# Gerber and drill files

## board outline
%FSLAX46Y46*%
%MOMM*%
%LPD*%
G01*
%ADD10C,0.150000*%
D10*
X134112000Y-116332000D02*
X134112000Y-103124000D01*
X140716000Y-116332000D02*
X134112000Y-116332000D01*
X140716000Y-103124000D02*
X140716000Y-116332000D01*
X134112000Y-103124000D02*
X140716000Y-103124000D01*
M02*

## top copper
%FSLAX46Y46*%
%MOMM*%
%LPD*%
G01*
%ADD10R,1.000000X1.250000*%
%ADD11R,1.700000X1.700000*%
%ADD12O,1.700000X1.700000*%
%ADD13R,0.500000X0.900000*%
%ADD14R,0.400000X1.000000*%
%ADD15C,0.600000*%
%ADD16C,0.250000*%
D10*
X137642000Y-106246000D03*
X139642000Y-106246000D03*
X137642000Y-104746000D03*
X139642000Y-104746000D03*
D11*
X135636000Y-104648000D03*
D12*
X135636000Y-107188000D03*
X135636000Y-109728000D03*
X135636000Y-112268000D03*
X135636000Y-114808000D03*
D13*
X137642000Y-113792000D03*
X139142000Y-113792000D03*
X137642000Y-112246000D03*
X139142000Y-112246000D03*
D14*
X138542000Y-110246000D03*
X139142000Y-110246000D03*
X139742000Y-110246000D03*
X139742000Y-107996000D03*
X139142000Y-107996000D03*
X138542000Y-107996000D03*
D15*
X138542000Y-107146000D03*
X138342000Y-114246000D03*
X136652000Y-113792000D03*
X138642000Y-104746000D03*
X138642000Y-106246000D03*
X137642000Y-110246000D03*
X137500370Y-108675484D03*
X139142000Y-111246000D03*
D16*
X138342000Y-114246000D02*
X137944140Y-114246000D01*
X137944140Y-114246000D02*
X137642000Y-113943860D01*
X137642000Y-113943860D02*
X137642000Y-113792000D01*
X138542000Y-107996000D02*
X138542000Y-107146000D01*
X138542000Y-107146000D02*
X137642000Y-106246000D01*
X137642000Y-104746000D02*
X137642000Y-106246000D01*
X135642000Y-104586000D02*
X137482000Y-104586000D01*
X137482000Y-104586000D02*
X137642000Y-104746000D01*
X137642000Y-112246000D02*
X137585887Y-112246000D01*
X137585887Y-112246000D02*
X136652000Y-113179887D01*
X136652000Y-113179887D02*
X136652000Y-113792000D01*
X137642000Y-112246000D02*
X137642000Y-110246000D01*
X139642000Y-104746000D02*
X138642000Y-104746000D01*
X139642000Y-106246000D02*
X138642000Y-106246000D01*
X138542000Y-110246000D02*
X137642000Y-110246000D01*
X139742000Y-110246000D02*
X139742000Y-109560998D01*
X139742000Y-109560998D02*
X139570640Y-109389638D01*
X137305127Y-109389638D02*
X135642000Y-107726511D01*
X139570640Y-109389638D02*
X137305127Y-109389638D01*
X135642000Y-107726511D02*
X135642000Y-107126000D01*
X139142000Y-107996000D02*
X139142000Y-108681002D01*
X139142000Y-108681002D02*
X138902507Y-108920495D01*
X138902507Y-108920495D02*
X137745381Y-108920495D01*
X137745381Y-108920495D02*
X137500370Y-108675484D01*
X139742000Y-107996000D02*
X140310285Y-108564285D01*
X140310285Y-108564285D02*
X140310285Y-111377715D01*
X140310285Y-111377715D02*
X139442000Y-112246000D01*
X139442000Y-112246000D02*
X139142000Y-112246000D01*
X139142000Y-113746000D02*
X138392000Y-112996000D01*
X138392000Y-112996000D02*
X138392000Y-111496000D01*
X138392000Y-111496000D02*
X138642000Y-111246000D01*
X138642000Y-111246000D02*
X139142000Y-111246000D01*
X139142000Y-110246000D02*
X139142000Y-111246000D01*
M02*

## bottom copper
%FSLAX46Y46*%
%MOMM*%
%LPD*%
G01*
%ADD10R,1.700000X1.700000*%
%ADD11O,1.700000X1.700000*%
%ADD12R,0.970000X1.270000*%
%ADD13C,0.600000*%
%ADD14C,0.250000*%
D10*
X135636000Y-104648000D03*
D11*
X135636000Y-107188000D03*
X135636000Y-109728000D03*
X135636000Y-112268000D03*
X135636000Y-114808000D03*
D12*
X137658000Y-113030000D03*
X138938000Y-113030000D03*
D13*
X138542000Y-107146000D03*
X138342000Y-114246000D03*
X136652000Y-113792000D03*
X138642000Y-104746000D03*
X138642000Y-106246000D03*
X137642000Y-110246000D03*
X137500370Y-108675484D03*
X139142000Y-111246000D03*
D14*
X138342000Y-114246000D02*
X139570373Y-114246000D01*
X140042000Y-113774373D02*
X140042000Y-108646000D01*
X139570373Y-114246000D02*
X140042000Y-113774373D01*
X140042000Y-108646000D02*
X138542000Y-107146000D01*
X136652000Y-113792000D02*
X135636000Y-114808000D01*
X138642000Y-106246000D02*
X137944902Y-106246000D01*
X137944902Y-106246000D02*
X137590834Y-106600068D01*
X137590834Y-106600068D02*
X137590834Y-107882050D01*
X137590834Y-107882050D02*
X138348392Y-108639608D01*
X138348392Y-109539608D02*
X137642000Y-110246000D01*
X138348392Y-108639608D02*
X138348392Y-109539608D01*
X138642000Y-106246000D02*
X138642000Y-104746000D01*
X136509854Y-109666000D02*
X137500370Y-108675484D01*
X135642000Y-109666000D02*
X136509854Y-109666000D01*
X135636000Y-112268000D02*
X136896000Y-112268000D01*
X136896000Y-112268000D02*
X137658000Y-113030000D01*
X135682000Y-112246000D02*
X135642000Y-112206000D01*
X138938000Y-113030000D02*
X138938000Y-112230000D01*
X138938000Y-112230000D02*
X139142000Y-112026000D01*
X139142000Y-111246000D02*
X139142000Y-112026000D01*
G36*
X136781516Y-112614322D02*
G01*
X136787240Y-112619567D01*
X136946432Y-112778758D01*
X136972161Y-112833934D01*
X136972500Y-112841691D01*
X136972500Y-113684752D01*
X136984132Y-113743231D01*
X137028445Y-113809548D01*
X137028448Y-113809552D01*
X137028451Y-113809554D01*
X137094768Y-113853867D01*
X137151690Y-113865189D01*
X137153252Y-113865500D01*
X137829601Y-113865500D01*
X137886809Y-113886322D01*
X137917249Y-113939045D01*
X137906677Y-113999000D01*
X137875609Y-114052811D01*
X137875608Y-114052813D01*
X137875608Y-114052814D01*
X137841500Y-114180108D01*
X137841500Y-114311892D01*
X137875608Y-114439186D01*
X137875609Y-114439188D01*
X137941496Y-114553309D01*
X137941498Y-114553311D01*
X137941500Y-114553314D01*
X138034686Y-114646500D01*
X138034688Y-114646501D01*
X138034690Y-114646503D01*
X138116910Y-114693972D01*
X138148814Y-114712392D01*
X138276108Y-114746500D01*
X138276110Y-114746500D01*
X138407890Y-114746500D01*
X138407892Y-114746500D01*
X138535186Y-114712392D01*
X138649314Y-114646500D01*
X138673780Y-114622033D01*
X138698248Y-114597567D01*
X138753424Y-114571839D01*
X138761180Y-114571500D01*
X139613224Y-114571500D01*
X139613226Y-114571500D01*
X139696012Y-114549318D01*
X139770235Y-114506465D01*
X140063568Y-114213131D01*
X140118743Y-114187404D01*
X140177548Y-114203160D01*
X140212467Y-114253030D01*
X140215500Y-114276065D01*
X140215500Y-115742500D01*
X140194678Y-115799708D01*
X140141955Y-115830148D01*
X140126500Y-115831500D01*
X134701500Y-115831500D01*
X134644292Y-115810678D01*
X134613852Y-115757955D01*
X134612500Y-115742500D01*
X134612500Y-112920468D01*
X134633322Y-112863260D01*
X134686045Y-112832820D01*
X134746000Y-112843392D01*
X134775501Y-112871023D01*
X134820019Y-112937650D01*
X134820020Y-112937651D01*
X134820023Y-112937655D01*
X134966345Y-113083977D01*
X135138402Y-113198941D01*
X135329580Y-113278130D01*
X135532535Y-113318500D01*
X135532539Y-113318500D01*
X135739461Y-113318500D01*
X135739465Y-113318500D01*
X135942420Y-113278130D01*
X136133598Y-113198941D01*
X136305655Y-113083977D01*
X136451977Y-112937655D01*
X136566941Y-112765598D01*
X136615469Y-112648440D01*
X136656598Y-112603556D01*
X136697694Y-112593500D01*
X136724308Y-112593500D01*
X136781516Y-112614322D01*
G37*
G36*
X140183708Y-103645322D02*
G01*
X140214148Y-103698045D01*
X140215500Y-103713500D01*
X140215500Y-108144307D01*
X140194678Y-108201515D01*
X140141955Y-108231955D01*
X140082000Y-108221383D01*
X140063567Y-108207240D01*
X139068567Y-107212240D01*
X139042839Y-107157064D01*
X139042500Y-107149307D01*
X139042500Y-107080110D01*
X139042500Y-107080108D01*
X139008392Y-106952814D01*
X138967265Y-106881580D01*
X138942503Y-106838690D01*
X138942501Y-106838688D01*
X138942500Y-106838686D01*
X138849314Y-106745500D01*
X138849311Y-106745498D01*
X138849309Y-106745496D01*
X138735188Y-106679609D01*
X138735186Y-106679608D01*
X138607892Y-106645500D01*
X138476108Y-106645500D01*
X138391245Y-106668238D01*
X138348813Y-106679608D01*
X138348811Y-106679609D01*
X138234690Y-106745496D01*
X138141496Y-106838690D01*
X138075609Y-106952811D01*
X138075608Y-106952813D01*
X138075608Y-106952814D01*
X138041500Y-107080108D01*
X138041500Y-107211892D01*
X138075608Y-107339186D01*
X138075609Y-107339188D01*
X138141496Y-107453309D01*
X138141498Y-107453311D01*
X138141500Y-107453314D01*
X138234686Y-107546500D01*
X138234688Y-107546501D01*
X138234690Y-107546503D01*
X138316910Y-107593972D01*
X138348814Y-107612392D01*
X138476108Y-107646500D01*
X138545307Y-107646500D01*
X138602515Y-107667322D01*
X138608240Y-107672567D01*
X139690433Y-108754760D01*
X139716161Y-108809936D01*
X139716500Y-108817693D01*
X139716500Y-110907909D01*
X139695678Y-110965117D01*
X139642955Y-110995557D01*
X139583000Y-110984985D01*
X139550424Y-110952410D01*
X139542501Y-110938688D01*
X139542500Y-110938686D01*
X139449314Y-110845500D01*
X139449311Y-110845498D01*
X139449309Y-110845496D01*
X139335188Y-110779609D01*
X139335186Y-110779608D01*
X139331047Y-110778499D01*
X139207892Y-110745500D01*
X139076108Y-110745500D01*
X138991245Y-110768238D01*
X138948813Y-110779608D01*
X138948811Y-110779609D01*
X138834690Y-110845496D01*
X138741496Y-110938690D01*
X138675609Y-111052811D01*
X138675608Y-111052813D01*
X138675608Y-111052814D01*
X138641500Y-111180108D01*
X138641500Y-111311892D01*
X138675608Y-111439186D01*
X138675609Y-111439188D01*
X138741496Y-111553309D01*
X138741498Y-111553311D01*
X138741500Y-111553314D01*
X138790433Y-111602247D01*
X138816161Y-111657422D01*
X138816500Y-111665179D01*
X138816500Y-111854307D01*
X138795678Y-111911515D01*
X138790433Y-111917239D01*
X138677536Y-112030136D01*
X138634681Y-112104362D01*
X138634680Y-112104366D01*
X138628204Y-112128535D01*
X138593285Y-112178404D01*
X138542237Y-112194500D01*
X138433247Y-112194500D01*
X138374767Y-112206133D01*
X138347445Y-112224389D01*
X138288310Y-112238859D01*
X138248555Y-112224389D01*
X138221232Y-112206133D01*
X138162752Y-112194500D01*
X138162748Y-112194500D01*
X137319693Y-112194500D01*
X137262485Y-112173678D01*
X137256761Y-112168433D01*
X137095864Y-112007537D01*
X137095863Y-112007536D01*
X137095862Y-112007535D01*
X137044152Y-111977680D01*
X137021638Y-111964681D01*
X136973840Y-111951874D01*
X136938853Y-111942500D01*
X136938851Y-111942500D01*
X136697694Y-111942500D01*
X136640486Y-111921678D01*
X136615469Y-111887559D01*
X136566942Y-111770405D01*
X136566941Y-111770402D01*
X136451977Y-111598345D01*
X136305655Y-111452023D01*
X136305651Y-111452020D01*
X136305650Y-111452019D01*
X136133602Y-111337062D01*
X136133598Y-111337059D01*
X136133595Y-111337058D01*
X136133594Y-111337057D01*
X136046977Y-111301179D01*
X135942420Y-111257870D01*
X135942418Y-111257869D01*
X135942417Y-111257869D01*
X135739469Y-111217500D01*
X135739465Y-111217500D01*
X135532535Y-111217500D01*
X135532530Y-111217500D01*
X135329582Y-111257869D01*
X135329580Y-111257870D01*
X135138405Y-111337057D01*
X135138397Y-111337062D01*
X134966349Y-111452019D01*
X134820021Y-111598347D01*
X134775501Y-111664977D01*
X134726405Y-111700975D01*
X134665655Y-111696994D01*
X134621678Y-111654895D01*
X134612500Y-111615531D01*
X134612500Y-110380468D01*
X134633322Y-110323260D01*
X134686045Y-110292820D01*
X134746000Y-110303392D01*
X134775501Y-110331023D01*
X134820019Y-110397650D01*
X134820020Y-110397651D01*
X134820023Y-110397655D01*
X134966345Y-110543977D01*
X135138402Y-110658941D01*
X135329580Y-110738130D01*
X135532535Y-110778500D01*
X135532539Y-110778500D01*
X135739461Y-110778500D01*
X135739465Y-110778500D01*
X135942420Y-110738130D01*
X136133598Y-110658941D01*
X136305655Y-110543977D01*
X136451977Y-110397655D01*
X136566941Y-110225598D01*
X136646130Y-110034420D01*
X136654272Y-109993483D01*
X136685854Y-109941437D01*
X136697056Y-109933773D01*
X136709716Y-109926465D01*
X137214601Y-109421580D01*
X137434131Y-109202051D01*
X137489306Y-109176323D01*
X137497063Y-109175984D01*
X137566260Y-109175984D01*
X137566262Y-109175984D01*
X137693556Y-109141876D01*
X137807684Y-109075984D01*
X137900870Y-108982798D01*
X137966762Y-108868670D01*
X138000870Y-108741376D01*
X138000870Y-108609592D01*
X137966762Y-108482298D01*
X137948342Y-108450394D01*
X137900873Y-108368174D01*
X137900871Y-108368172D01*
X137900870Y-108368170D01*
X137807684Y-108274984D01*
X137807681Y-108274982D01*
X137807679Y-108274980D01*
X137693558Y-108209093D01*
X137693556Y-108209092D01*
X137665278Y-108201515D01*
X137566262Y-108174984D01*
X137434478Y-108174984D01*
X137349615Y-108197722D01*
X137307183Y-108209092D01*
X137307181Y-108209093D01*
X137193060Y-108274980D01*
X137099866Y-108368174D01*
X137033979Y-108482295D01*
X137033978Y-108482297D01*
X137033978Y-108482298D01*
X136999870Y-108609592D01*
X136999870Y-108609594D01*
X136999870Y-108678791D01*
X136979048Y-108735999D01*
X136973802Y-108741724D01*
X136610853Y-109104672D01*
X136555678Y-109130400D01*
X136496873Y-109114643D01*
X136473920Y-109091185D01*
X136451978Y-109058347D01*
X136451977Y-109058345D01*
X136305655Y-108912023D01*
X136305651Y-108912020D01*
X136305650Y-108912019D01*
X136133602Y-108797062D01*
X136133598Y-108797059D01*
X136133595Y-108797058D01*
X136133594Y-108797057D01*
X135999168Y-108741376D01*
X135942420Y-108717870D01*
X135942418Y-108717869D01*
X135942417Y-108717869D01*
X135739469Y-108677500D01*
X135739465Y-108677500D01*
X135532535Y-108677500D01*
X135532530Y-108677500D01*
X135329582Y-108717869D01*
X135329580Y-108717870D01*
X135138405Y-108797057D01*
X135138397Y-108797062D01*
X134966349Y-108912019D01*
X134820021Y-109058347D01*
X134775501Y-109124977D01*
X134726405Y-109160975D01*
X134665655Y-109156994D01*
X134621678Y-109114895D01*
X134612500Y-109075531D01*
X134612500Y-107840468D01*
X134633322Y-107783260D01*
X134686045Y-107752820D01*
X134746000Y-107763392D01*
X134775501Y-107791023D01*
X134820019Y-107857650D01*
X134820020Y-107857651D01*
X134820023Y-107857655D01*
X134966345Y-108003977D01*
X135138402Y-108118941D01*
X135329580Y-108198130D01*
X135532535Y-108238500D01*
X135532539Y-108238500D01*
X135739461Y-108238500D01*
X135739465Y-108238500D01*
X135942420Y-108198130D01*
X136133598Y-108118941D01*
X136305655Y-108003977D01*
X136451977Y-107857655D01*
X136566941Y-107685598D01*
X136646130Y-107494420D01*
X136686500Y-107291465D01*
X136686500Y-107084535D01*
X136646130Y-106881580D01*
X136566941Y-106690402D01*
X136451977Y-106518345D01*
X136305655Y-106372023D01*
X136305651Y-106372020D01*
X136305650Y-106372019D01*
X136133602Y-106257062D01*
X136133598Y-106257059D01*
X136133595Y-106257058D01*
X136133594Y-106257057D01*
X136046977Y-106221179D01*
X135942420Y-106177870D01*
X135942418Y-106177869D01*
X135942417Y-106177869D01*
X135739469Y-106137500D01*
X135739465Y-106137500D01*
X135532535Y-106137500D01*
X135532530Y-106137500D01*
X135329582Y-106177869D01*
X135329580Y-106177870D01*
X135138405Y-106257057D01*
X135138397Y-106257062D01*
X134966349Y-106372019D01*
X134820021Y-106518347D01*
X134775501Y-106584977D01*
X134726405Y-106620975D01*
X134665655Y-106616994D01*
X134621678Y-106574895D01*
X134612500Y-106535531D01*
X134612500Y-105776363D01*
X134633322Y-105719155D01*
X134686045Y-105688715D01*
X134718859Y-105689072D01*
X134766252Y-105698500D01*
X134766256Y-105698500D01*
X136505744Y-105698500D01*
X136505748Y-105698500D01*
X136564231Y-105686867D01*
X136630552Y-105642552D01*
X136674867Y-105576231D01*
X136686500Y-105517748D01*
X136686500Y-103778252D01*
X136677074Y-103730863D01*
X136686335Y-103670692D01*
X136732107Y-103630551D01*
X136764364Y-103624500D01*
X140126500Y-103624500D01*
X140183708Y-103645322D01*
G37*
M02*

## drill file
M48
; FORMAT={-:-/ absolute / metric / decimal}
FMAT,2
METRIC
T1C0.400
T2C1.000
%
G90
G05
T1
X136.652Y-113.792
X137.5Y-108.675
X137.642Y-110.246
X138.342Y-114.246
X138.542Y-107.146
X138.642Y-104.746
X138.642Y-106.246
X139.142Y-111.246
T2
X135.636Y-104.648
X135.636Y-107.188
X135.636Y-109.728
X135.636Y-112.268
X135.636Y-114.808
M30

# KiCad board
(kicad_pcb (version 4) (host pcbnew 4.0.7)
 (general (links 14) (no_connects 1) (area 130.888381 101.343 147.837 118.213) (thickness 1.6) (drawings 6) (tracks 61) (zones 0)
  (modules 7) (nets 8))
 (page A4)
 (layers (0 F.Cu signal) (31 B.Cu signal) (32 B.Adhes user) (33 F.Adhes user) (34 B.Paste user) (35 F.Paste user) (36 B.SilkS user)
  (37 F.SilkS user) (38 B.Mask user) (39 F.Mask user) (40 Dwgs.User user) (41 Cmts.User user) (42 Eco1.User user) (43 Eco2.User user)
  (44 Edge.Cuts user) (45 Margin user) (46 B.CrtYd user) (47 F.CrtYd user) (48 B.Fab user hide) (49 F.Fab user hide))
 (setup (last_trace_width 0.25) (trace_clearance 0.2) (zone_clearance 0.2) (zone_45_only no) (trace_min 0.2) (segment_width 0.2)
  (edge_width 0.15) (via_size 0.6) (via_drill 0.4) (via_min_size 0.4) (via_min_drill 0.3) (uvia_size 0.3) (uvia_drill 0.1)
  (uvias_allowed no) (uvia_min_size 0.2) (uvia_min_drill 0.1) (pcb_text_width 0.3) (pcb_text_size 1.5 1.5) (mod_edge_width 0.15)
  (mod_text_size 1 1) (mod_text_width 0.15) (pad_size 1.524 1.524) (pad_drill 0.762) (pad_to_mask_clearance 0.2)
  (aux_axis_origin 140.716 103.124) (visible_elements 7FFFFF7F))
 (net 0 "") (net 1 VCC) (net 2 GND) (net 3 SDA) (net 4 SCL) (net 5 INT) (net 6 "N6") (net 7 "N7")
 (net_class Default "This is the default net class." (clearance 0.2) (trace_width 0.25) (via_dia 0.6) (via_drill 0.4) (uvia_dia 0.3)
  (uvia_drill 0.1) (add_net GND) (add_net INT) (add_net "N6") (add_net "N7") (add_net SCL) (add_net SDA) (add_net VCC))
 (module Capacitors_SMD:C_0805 (layer F.Cu) (at 138.642 106.246)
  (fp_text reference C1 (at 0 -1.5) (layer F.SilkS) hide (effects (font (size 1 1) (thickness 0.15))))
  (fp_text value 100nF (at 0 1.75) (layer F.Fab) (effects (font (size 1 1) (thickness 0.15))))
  (pad 1 smd rect (at -1 0) (size 1 1.25) (layers F.Cu F.Paste F.Mask) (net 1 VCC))
  (pad 2 smd rect (at 1 0) (size 1 1.25) (layers F.Cu F.Paste F.Mask) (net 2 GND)))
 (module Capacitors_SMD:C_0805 (layer F.Cu) (at 138.642 104.746)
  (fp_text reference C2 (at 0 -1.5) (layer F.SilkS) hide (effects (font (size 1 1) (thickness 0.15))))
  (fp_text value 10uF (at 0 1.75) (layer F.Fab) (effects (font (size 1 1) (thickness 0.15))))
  (pad 1 smd rect (at -1 0) (size 1 1.25) (layers F.Cu F.Paste F.Mask) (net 1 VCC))
  (pad 2 smd rect (at 1 0) (size 1 1.25) (layers F.Cu F.Paste F.Mask) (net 2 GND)))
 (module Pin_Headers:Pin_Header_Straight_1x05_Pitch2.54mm (layer F.Cu) (at 135.636 104.648)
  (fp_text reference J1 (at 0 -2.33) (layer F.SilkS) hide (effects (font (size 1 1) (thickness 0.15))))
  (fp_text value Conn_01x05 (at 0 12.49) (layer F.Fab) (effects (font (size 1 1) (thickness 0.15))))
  (pad 1 thru_hole rect (at 0 0) (size 1.7 1.7) (drill 1) (layers *.Cu *.Mask) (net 1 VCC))
  (pad 2 thru_hole oval (at 0 2.54) (size 1.7 1.7) (drill 1) (layers *.Cu *.Mask) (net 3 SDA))
  (pad 3 thru_hole oval (at 0 5.08) (size 1.7 1.7) (drill 1) (layers *.Cu *.Mask) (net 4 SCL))
  (pad 4 thru_hole oval (at 0 7.62) (size 1.7 1.7) (drill 1) (layers *.Cu *.Mask) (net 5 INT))
  (pad 5 thru_hole oval (at 0 10.16) (size 1.7 1.7) (drill 1) (layers *.Cu *.Mask) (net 2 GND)))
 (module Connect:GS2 (layer B.Cu) (at 138.298 113.03 270)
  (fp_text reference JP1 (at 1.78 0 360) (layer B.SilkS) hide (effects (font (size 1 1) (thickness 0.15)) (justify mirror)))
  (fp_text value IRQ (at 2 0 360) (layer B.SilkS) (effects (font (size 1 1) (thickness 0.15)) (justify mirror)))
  (pad 1 smd rect (at 0 0.64 270) (size 1.27 0.97) (layers B.Cu B.Paste B.Mask) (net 5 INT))
  (pad 2 smd rect (at 0 -0.64 270) (size 1.27 0.97) (layers B.Cu B.Paste B.Mask) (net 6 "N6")))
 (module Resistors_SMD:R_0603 (layer F.Cu) (at 138.392 113.792)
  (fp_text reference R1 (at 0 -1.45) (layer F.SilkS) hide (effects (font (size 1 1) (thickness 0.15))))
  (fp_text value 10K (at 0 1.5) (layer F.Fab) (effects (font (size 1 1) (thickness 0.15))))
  (pad 1 smd rect (at -0.75 0) (size 0.5 0.9) (layers F.Cu F.Paste F.Mask) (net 1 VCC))
  (pad 2 smd rect (at 0.75 0) (size 0.5 0.9) (layers F.Cu F.Paste F.Mask) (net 6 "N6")))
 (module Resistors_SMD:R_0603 (layer F.Cu) (at 138.392 112.246)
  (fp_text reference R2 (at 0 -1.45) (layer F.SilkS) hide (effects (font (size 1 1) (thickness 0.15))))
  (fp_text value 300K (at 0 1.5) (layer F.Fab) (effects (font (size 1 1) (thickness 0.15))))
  (pad 1 smd rect (at -0.75 0) (size 0.5 0.9) (layers F.Cu F.Paste F.Mask) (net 2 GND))
  (pad 2 smd rect (at 0.75 0) (size 0.5 0.9) (layers F.Cu F.Paste F.Mask) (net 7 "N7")))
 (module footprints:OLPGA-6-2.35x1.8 (layer F.Cu) (at 139.142 109.171 90)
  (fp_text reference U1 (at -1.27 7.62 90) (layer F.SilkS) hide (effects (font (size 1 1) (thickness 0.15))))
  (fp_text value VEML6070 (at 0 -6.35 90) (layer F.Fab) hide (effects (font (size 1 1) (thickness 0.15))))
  (pad 1 smd rect (at -1.075 -0.6 90) (size 1 0.4) (layers F.Cu F.Paste F.Mask) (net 2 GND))
  (pad 2 smd rect (at -1.075 0 90) (size 1 0.4) (layers F.Cu F.Paste F.Mask) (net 6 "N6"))
  (pad 3 smd rect (at -1.075 0.6 90) (size 1 0.4) (layers F.Cu F.Paste F.Mask) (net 3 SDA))
  (pad 4 smd rect (at 1.175 0.6 90) (size 1 0.4) (layers F.Cu F.Paste F.Mask) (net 7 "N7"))
  (pad 5 smd rect (at 1.175 0 90) (size 1 0.4) (layers F.Cu F.Paste F.Mask) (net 4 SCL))
  (pad 6 smd rect (at 1.175 -0.6 90) (size 1 0.4) (layers F.Cu F.Paste F.Mask) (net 1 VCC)))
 (gr_line (start 134.112 116.332) (end 134.112 103.124) (layer Edge.Cuts) (width 0.15))
 (gr_line (start 140.716 116.332) (end 134.112 116.332) (layer Edge.Cuts) (width 0.15))
 (gr_line (start 140.716 103.124) (end 140.716 116.332) (layer Edge.Cuts) (width 0.15))
 (gr_line (start 134.112 103.124) (end 140.716 103.124) (layer Edge.Cuts) (width 0.15))
 (segment (start 138.342 114.246) (end 137.94414 114.246) (width 0.25) (layer F.Cu) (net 1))
 (segment (start 137.94414 114.246) (end 137.642 113.94386) (width 0.25) (layer F.Cu) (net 1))
 (segment (start 137.642 113.94386) (end 137.642 113.792) (width 0.25) (layer F.Cu) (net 1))
 (segment (start 138.342 114.246) (end 139.570373 114.246) (width 0.25) (layer B.Cu) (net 1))
 (segment (start 140.042 113.774373) (end 140.042 108.646) (width 0.25) (layer B.Cu) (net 1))
 (segment (start 139.570373 114.246) (end 140.042 113.774373) (width 0.25) (layer B.Cu) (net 1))
 (segment (start 140.042 108.646) (end 138.542 107.146) (width 0.25) (layer B.Cu) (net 1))
 (via (at 138.542 107.146) (size 0.6) (drill 0.4) (layers F.Cu B.Cu) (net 1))
 (via (at 138.342 114.246) (size 0.6) (drill 0.4) (layers F.Cu B.Cu) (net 1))
 (segment (start 138.542 107.996) (end 138.542 107.146) (width 0.25) (layer F.Cu) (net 1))
 (segment (start 138.542 107.146) (end 137.642 106.246) (width 0.25) (layer F.Cu) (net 1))
 (segment (start 137.642 104.746) (end 137.642 106.246) (width 0.25) (layer F.Cu) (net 1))
 (segment (start 135.642 104.586) (end 137.482 104.586) (width 0.25) (layer F.Cu) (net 1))
 (segment (start 137.482 104.586) (end 137.642 104.746) (width 0.25) (layer F.Cu) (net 1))
 (segment (start 137.642 112.246) (end 137.585887 112.246) (width 0.25) (layer F.Cu) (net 2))
 (segment (start 137.585887 112.246) (end 136.652 113.179887) (width 0.25) (layer F.Cu) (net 2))
 (segment (start 136.652 113.179887) (end 136.652 113.792) (width 0.25) (layer F.Cu) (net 2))
 (segment (start 136.652 113.792) (end 135.636 114.808) (width 0.25) (layer B.Cu) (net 2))
 (via (at 136.652 113.792) (size 0.6) (drill 0.4) (layers F.Cu B.Cu) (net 2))
 (segment (start 137.642 112.246) (end 137.642 110.246) (width 0.25) (layer F.Cu) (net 2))
 (segment (start 138.642 106.246) (end 137.944902 106.246) (width 0.25) (layer B.Cu) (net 2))
 (segment (start 137.944902 106.246) (end 137.590834 106.600068) (width 0.25) (layer B.Cu) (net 2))
 (segment (start 137.590834 106.600068) (end 137.590834 107.88205) (width 0.25) (layer B.Cu) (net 2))
 (segment (start 137.590834 107.88205) (end 138.348392 108.639608) (width 0.25) (layer B.Cu) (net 2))
 (segment (start 138.348392 109.539608) (end 137.642 110.246) (width 0.25) (layer B.Cu) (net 2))
 (segment (start 138.348392 108.639608) (end 138.348392 109.539608) (width 0.25) (layer B.Cu) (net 2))
 (segment (start 139.642 104.746) (end 138.642 104.746) (width 0.25) (layer F.Cu) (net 2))
 (via (at 138.642 104.746) (size 0.6) (drill 0.4) (layers F.Cu B.Cu) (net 2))
 (segment (start 138.642 106.246) (end 138.642 104.746) (width 0.25) (layer B.Cu) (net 2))
 (segment (start 139.642 106.246) (end 138.642 106.246) (width 0.25) (layer F.Cu) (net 2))
 (via (at 138.642 106.246) (size 0.6) (drill 0.4) (layers F.Cu B.Cu) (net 2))
 (segment (start 138.542 110.246) (end 137.642 110.246) (width 0.25) (layer F.Cu) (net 2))
 (via (at 137.642 110.246) (size 0.6) (drill 0.4) (layers F.Cu B.Cu) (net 2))
 (segment (start 139.742 110.246) (end 139.742 109.560998) (width 0.25) (layer F.Cu) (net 3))
 (segment (start 139.742 109.560998) (end 139.57064 109.389638) (width 0.25) (layer F.Cu) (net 3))
 (segment (start 137.305127 109.389638) (end 135.642 107.726511) (width 0.25) (layer F.Cu) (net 3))
 (segment (start 139.57064 109.389638) (end 137.305127 109.389638) (width 0.25) (layer F.Cu) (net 3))
 (segment (start 135.642 107.726511) (end 135.642 107.126) (width 0.25) (layer F.Cu) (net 3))
 (segment (start 139.142 107.996) (end 139.142 108.681002) (width 0.25) (layer F.Cu) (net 4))
 (segment (start 139.142 108.681002) (end 138.902507 108.920495) (width 0.25) (layer F.Cu) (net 4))
 (segment (start 138.902507 108.920495) (end 137.745381 108.920495) (width 0.25) (layer F.Cu) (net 4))
 (segment (start 137.745381 108.920495) (end 137.50037 108.675484) (width 0.25) (layer F.Cu) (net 4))
 (segment (start 136.509854 109.666) (end 137.50037 108.675484) (width 0.25) (layer B.Cu) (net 4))
 (via (at 137.50037 108.675484) (size 0.6) (drill 0.4) (layers F.Cu B.Cu) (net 4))
 (segment (start 135.642 109.666) (end 136.509854 109.666) (width 0.25) (layer B.Cu) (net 4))
 (segment (start 135.636 112.268) (end 136.896 112.268) (width 0.25) (layer B.Cu) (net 5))
 (segment (start 136.896 112.268) (end 137.658 113.03) (width 0.25) (layer B.Cu) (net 5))
 (segment (start 135.682 112.246) (end 135.642 112.206) (width 0.25) (layer B.Cu) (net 5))
 (segment (start 139.742 107.996) (end 140.310285 108.564285) (width 0.25) (layer F.Cu) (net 7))
 (segment (start 140.310285 108.564285) (end 140.310285 111.377715) (width 0.25) (layer F.Cu) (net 7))
 (segment (start 140.310285 111.377715) (end 139.442 112.246) (width 0.25) (layer F.Cu) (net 7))
 (segment (start 139.442 112.246) (end 139.142 112.246) (width 0.25) (layer F.Cu) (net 7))
 (segment (start 138.938 113.03) (end 138.938 112.23) (width 0.25) (layer B.Cu) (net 6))
 (segment (start 138.938 112.23) (end 139.142 112.026) (width 0.25) (layer B.Cu) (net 6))
 (segment (start 139.142 113.746) (end 138.392 112.996) (width 0.25) (layer F.Cu) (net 6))
 (segment (start 138.392 112.996) (end 138.392 111.496) (width 0.25) (layer F.Cu) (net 6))
 (segment (start 138.392 111.496) (end 138.642 111.246) (width 0.25) (layer F.Cu) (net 6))
 (segment (start 138.642 111.246) (end 139.142 111.246) (width 0.25) (layer F.Cu) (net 6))
 (segment (start 139.142 111.246) (end 139.142 112.026) (width 0.25) (layer B.Cu) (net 6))
 (segment (start 139.142 110.246) (end 139.142 111.246) (width 0.25) (layer F.Cu) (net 6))
 (via (at 139.142 111.246) (size 0.6) (drill 0.4) (layers F.Cu B.Cu) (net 6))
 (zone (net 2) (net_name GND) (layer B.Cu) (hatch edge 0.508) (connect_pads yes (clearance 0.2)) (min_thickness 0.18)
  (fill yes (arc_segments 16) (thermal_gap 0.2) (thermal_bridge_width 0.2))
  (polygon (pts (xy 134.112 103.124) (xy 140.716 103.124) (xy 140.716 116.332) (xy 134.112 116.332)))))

